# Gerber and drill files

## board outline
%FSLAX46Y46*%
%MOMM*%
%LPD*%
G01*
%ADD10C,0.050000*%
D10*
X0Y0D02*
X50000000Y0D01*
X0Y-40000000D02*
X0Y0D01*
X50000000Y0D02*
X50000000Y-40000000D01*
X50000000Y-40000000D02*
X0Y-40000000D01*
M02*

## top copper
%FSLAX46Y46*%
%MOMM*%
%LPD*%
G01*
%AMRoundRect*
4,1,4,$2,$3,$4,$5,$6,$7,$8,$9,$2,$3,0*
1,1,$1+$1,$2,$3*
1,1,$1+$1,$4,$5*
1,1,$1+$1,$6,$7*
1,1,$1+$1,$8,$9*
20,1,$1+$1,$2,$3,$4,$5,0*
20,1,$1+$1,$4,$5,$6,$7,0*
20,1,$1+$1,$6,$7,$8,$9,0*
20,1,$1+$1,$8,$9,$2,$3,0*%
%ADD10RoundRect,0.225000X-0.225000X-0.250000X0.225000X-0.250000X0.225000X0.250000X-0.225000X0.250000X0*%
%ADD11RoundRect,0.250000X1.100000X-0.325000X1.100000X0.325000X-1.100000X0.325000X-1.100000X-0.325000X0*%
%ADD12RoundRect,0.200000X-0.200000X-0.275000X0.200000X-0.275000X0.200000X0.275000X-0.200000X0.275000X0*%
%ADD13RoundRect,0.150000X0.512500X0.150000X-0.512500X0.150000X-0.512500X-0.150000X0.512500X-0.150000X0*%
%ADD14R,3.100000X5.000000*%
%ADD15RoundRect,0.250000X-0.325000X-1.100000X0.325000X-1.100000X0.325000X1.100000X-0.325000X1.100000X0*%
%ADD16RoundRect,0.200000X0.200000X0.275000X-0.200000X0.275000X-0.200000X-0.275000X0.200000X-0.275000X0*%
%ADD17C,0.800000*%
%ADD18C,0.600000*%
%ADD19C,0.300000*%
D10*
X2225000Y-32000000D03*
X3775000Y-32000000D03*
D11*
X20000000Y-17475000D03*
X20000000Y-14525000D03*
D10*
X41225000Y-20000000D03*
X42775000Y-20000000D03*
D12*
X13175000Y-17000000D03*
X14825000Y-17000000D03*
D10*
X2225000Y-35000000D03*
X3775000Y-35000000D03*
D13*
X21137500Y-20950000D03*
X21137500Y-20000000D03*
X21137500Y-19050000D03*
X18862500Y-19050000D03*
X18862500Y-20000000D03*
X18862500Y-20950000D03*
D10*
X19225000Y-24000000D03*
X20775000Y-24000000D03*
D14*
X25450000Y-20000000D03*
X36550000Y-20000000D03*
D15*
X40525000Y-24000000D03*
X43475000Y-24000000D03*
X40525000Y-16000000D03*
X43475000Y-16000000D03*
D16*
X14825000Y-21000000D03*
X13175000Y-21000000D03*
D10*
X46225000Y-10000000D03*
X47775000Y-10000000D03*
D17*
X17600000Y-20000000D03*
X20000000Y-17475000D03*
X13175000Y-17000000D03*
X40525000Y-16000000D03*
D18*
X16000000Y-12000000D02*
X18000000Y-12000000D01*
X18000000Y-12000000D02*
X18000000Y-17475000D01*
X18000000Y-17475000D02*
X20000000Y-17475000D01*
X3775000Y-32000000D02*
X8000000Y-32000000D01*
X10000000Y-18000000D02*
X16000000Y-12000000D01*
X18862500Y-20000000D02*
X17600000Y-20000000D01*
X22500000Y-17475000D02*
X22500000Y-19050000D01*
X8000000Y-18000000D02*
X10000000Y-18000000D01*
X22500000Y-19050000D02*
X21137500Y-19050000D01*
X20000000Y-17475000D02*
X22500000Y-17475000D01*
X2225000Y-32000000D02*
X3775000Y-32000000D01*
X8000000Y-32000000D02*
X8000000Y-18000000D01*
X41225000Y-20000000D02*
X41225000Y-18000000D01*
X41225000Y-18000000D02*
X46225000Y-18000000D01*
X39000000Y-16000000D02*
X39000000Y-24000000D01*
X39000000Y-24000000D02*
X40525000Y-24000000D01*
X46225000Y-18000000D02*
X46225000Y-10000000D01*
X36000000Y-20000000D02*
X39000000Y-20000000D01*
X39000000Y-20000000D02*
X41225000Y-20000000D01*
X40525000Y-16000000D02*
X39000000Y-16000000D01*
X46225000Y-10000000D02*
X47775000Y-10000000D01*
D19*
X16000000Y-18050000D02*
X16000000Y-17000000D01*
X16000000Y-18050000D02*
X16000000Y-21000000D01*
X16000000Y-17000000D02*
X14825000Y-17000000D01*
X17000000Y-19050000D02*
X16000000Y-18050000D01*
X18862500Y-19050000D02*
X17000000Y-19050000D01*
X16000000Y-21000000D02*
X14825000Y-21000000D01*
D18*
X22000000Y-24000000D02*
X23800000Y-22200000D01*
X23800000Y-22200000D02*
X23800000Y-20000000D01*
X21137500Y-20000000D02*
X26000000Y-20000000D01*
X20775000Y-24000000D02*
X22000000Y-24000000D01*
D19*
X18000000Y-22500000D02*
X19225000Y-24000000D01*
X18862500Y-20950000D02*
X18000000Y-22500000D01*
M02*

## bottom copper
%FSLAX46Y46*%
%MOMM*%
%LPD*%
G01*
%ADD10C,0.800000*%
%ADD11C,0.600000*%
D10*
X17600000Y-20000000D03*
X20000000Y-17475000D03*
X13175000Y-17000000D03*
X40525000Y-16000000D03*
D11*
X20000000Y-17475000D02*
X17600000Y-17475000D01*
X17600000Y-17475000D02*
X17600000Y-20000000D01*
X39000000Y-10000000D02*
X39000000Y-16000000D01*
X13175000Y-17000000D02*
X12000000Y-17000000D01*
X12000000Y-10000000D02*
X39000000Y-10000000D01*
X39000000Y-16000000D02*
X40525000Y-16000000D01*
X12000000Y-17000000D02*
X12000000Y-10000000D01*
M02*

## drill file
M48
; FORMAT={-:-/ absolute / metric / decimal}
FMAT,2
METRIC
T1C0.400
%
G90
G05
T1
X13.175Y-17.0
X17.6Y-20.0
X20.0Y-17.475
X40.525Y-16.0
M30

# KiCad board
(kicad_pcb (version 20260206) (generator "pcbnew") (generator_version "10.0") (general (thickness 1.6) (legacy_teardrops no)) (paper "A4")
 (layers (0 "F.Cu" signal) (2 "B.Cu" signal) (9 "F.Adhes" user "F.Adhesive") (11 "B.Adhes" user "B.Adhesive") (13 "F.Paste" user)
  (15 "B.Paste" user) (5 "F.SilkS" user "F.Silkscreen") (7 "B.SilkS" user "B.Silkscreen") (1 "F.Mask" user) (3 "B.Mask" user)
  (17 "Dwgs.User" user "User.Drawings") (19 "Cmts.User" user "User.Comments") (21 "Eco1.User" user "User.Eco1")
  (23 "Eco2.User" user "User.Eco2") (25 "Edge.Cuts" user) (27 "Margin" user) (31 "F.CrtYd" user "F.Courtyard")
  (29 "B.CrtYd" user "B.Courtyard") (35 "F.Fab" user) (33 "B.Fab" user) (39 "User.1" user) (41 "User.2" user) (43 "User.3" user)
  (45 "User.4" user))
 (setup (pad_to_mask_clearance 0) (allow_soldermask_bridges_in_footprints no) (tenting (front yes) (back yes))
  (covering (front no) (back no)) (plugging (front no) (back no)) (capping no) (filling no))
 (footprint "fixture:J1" (layer "F.Cu") (at 3 32)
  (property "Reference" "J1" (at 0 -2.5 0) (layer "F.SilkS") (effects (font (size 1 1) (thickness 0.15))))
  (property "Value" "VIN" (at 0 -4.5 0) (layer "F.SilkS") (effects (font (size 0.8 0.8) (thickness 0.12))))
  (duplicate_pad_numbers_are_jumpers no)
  (pad "1" smd roundrect (at -0.775 0) (size 0.9 0.95) (layers "F.Cu" "F.Mask" "F.Paste") (roundrect_rratio 0.25) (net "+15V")
   (thermal_bridge_angle 45))
  (pad "2" smd roundrect (at 0.775 0) (size 0.9 0.95) (layers "F.Cu" "F.Mask" "F.Paste") (roundrect_rratio 0.25) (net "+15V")
   (thermal_bridge_angle 45)))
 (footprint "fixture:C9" (layer "F.Cu") (at 20 16 90)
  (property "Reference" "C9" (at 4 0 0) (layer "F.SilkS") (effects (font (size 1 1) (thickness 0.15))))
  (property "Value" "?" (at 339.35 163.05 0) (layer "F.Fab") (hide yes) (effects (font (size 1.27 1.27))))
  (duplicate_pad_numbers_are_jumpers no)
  (pad "1" smd roundrect (at -1.475 0 90) (size 1.15 2.7) (layers "F.Cu" "F.Mask" "F.Paste") (roundrect_rratio 0.217391) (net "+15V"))
  (pad "2" smd roundrect (at 1.475 0 90) (size 1.15 2.7) (layers "F.Cu" "F.Mask" "F.Paste") (roundrect_rratio 0.217391) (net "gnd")))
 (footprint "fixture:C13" (layer "F.Cu") (at 42 20)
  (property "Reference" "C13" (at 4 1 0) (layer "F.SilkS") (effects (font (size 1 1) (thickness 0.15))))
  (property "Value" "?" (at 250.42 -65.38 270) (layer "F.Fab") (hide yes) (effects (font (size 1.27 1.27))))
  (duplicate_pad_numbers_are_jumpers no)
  (pad "1" smd roundrect (at -0.775 0) (size 0.9 0.95) (layers "F.Cu" "F.Mask" "F.Paste") (roundrect_rratio 0.25) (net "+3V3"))
  (pad "2" smd roundrect (at 0.775 0) (size 0.9 0.95) (layers "F.Cu" "F.Mask" "F.Paste") (roundrect_rratio 0.25) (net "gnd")))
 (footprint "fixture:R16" (layer "F.Cu") (at 14 17)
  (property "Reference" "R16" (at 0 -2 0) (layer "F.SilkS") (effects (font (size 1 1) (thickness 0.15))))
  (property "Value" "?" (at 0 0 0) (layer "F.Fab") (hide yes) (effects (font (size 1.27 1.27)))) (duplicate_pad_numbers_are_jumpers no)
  (pad "1" smd roundrect (at -0.825 0) (size 0.8 0.95) (layers "F.Cu" "F.Mask" "F.Paste") (roundrect_rratio 0.25) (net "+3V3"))
  (pad "2" smd roundrect (at 0.825 0) (size 0.8 0.95) (layers "F.Cu" "F.Mask" "F.Paste") (roundrect_rratio 0.25) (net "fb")))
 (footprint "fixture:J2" (layer "F.Cu") (at 3 35)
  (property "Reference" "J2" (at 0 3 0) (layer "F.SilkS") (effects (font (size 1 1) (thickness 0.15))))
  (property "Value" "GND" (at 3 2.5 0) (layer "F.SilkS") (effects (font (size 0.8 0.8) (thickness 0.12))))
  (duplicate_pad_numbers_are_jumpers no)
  (pad "1" smd roundrect (at -0.775 0) (size 0.9 0.95) (layers "F.Cu" "F.Mask" "F.Paste") (roundrect_rratio 0.25) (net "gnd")
   (thermal_bridge_angle 45))
  (pad "2" smd roundrect (at 0.775 0) (size 0.9 0.95) (layers "F.Cu" "F.Mask" "F.Paste") (roundrect_rratio 0.25) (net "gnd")
   (thermal_bridge_angle 45)))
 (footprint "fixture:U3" (layer "F.Cu") (at 20 20 180)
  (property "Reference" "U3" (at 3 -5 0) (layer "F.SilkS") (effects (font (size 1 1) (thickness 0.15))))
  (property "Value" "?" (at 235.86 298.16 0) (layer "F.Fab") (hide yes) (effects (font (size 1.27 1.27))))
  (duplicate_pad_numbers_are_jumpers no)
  (pad "1" smd roundrect (at -1.1375 -0.95 180) (size 1.325 0.6) (layers "F.Cu" "F.Mask" "F.Paste") (roundrect_rratio 0.25) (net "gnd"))
  (pad "2" smd roundrect (at -1.1375 0 180) (size 1.325 0.6) (layers "F.Cu" "F.Mask" "F.Paste") (roundrect_rratio 0.25) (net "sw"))
  (pad "3" smd roundrect (at -1.1375 0.95 180) (size 1.325 0.6) (layers "F.Cu" "F.Mask" "F.Paste") (roundrect_rratio 0.25) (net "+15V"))
  (pad "4" smd roundrect (at 1.1375 0.95 180) (size 1.325 0.6) (layers "F.Cu" "F.Mask" "F.Paste") (roundrect_rratio 0.25) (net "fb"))
  (pad "5" smd roundrect (at 1.1375 0 180) (size 1.325 0.6) (layers "F.Cu" "F.Mask" "F.Paste") (roundrect_rratio 0.25) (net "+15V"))
  (pad "6" smd roundrect (at 1.1375 -0.95 180) (size 1.325 0.6) (layers "F.Cu" "F.Mask" "F.Paste") (roundrect_rratio 0.25) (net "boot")))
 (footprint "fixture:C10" (layer "F.Cu") (at 20 24)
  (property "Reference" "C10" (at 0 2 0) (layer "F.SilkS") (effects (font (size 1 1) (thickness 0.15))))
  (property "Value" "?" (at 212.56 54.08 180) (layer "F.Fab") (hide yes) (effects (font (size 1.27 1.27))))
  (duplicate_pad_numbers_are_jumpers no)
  (pad "1" smd roundrect (at -0.775 0) (size 0.9 0.95) (layers "F.Cu" "F.Mask" "F.Paste") (roundrect_rratio 0.25) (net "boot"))
  (pad "2" smd roundrect (at 0.775 0) (size 0.9 0.95) (layers "F.Cu" "F.Mask" "F.Paste") (roundrect_rratio 0.25) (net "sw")))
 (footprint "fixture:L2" (layer "F.Cu") (at 31 20)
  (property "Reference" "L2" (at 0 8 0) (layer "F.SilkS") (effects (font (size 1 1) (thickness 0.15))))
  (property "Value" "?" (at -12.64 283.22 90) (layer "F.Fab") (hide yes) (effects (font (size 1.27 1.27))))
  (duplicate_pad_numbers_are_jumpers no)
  (pad "1" smd rect (at -5.55 0) (size 3.1 5) (layers "F.Cu" "F.Mask" "F.Paste") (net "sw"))
  (pad "2" smd rect (at 5.55 0) (size 3.1 5) (layers "F.Cu" "F.Mask" "F.Paste") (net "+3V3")))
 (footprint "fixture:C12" (layer "F.Cu") (at 42 24)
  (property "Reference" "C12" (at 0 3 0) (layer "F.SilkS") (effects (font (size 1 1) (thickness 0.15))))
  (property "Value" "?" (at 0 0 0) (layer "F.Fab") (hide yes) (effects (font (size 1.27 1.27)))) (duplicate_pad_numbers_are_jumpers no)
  (pad "1" smd roundrect (at -1.475 0) (size 1.15 2.7) (layers "F.Cu" "F.Mask" "F.Paste") (roundrect_rratio 0.217391) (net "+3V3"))
  (pad "2" smd roundrect (at 1.475 0) (size 1.15 2.7) (layers "F.Cu" "F.Mask" "F.Paste") (roundrect_rratio 0.217391) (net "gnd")))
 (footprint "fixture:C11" (layer "F.Cu") (at 42 16)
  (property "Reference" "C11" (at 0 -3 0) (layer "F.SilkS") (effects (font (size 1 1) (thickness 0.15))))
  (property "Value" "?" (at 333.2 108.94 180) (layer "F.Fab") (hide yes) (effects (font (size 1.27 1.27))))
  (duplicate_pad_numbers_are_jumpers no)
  (pad "1" smd roundrect (at -1.475 0) (size 1.15 2.7) (layers "F.Cu" "F.Mask" "F.Paste") (roundrect_rratio 0.217391) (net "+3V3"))
  (pad "2" smd roundrect (at 1.475 0) (size 1.15 2.7) (layers "F.Cu" "F.Mask" "F.Paste") (roundrect_rratio 0.217391) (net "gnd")))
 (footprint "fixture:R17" (layer "F.Cu") (at 14 21 180)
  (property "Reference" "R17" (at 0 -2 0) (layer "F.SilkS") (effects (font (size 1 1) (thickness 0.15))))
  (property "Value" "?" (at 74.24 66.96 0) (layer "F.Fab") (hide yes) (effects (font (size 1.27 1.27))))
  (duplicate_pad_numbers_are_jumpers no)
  (pad "1" smd roundrect (at -0.825 0 180) (size 0.8 0.95) (layers "F.Cu" "F.Mask" "F.Paste") (roundrect_rratio 0.25) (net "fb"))
  (pad "2" smd roundrect (at 0.825 0 180) (size 0.8 0.95) (layers "F.Cu" "F.Mask" "F.Paste") (roundrect_rratio 0.25) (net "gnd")))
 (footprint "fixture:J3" (layer "F.Cu") (at 47 10)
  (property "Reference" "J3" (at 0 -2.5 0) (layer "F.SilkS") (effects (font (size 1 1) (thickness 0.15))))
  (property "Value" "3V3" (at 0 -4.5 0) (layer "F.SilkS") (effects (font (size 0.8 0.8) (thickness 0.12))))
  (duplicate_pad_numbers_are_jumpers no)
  (pad "1" smd roundrect (at -0.775 0) (size 0.9 0.95) (layers "F.Cu" "F.Mask" "F.Paste") (roundrect_rratio 0.25) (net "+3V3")
   (thermal_bridge_angle 45))
  (pad "2" smd roundrect (at 0.775 0) (size 0.9 0.95) (layers "F.Cu" "F.Mask" "F.Paste") (roundrect_rratio 0.25) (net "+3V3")
   (thermal_bridge_angle 45)))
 (gr_line (start 0 0) (end 50 0) (stroke (width 0.05) (type default)) (layer "Edge.Cuts"))
 (gr_line (start 0 40) (end 0 0) (stroke (width 0.05) (type default)) (layer "Edge.Cuts"))
 (gr_line (start 50 0) (end 50 40) (stroke (width 0.05) (type default)) (layer "Edge.Cuts"))
 (gr_line (start 50 40) (end 0 40) (stroke (width 0.05) (type default)) (layer "Edge.Cuts"))
 (segment (start 16 12) (end 18 12) (width 0.6) (layer "F.Cu") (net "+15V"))
 (segment (start 18 12) (end 18 17.475) (width 0.6) (layer "F.Cu") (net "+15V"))
 (segment (start 18 17.475) (end 20 17.475) (width 0.6) (layer "F.Cu") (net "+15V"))
 (segment (start 3.775 32) (end 8 32) (width 0.6) (layer "F.Cu") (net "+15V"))
 (segment (start 10 18) (end 16 12) (width 0.6) (layer "F.Cu") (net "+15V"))
 (segment (start 18.8625 20) (end 17.6 20) (width 0.6) (layer "F.Cu") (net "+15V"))
 (segment (start 22.5 17.475) (end 22.5 19.05) (width 0.6) (layer "F.Cu") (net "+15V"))
 (segment (start 8 18) (end 10 18) (width 0.6) (layer "F.Cu") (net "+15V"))
 (segment (start 22.5 19.05) (end 21.1375 19.05) (width 0.6) (layer "F.Cu") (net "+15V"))
 (segment (start 20 17.475) (end 22.5 17.475) (width 0.6) (layer "F.Cu") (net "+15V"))
 (segment (start 2.225 32) (end 3.775 32) (width 0.6) (layer "F.Cu") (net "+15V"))
 (segment (start 8 32) (end 8 18) (width 0.6) (layer "F.Cu") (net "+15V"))
 (via (at 17.6 20) (size 0.8) (drill 0.4) (layers "F.Cu" "B.Cu") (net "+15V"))
 (via (at 20 17.475) (size 0.8) (drill 0.4) (layers "F.Cu" "B.Cu") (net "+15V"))
 (segment (start 20 17.475) (end 17.6 17.475) (width 0.6) (layer "B.Cu") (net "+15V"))
 (segment (start 17.6 17.475) (end 17.6 20) (width 0.6) (layer "B.Cu") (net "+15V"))
 (segment (start 41.225 20) (end 41.225 18) (width 0.6) (layer "F.Cu") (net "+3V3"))
 (segment (start 41.225 18) (end 46.225 18) (width 0.6) (layer "F.Cu") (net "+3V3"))
 (segment (start 39 16) (end 39 24) (width 0.6) (layer "F.Cu") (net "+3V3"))
 (segment (start 39 24) (end 40.525 24) (width 0.6) (layer "F.Cu") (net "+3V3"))
 (segment (start 46.225 18) (end 46.225 10) (width 0.6) (layer "F.Cu") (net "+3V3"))
 (segment (start 36 20) (end 39 20) (width 0.6) (layer "F.Cu") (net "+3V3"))
 (segment (start 39 20) (end 41.225 20) (width 0.6) (layer "F.Cu") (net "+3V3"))
 (segment (start 40.525 16) (end 39 16) (width 0.6) (layer "F.Cu") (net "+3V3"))
 (segment (start 46.225 10) (end 47.775 10) (width 0.6) (layer "F.Cu") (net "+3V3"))
 (via (at 13.175 17) (size 0.8) (drill 0.4) (layers "F.Cu" "B.Cu") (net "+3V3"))
 (via (at 40.525 16) (size 0.8) (drill 0.4) (layers "F.Cu" "B.Cu") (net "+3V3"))
 (segment (start 39 10) (end 39 16) (width 0.6) (layer "B.Cu") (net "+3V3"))
 (segment (start 13.175 17) (end 12 17) (width 0.6) (layer "B.Cu") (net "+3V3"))
 (segment (start 12 10) (end 39 10) (width 0.6) (layer "B.Cu") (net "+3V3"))
 (segment (start 39 16) (end 40.525 16) (width 0.6) (layer "B.Cu") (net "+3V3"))
 (segment (start 12 17) (end 12 10) (width 0.6) (layer "B.Cu") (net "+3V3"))
 (segment (start 16 18.05) (end 16 17) (width 0.3) (layer "F.Cu") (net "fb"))
 (segment (start 16 18.05) (end 16 21) (width 0.3) (layer "F.Cu") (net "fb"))
 (segment (start 16 17) (end 14.825 17) (width 0.3) (layer "F.Cu") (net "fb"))
 (segment (start 17 19.05) (end 16 18.05) (width 0.3) (layer "F.Cu") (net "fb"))
 (segment (start 18.8625 19.05) (end 17 19.05) (width 0.3) (layer "F.Cu") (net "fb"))
 (segment (start 16 21) (end 14.825 21) (width 0.3) (layer "F.Cu") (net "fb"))
 (segment (start 22 24) (end 23.8 22.2) (width 0.6) (layer "F.Cu") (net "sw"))
 (segment (start 23.8 22.2) (end 23.8 20) (width 0.6) (layer "F.Cu") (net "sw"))
 (segment (start 21.1375 20) (end 26 20) (width 0.6) (layer "F.Cu") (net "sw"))
 (segment (start 20.775 24) (end 22 24) (width 0.6) (layer "F.Cu") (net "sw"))
 (segment (start 18 22.5) (end 19.225 24) (width 0.3) (layer "F.Cu") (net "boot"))
 (segment (start 18.8625 20.95) (end 18 22.5) (width 0.3) (layer "F.Cu") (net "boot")))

